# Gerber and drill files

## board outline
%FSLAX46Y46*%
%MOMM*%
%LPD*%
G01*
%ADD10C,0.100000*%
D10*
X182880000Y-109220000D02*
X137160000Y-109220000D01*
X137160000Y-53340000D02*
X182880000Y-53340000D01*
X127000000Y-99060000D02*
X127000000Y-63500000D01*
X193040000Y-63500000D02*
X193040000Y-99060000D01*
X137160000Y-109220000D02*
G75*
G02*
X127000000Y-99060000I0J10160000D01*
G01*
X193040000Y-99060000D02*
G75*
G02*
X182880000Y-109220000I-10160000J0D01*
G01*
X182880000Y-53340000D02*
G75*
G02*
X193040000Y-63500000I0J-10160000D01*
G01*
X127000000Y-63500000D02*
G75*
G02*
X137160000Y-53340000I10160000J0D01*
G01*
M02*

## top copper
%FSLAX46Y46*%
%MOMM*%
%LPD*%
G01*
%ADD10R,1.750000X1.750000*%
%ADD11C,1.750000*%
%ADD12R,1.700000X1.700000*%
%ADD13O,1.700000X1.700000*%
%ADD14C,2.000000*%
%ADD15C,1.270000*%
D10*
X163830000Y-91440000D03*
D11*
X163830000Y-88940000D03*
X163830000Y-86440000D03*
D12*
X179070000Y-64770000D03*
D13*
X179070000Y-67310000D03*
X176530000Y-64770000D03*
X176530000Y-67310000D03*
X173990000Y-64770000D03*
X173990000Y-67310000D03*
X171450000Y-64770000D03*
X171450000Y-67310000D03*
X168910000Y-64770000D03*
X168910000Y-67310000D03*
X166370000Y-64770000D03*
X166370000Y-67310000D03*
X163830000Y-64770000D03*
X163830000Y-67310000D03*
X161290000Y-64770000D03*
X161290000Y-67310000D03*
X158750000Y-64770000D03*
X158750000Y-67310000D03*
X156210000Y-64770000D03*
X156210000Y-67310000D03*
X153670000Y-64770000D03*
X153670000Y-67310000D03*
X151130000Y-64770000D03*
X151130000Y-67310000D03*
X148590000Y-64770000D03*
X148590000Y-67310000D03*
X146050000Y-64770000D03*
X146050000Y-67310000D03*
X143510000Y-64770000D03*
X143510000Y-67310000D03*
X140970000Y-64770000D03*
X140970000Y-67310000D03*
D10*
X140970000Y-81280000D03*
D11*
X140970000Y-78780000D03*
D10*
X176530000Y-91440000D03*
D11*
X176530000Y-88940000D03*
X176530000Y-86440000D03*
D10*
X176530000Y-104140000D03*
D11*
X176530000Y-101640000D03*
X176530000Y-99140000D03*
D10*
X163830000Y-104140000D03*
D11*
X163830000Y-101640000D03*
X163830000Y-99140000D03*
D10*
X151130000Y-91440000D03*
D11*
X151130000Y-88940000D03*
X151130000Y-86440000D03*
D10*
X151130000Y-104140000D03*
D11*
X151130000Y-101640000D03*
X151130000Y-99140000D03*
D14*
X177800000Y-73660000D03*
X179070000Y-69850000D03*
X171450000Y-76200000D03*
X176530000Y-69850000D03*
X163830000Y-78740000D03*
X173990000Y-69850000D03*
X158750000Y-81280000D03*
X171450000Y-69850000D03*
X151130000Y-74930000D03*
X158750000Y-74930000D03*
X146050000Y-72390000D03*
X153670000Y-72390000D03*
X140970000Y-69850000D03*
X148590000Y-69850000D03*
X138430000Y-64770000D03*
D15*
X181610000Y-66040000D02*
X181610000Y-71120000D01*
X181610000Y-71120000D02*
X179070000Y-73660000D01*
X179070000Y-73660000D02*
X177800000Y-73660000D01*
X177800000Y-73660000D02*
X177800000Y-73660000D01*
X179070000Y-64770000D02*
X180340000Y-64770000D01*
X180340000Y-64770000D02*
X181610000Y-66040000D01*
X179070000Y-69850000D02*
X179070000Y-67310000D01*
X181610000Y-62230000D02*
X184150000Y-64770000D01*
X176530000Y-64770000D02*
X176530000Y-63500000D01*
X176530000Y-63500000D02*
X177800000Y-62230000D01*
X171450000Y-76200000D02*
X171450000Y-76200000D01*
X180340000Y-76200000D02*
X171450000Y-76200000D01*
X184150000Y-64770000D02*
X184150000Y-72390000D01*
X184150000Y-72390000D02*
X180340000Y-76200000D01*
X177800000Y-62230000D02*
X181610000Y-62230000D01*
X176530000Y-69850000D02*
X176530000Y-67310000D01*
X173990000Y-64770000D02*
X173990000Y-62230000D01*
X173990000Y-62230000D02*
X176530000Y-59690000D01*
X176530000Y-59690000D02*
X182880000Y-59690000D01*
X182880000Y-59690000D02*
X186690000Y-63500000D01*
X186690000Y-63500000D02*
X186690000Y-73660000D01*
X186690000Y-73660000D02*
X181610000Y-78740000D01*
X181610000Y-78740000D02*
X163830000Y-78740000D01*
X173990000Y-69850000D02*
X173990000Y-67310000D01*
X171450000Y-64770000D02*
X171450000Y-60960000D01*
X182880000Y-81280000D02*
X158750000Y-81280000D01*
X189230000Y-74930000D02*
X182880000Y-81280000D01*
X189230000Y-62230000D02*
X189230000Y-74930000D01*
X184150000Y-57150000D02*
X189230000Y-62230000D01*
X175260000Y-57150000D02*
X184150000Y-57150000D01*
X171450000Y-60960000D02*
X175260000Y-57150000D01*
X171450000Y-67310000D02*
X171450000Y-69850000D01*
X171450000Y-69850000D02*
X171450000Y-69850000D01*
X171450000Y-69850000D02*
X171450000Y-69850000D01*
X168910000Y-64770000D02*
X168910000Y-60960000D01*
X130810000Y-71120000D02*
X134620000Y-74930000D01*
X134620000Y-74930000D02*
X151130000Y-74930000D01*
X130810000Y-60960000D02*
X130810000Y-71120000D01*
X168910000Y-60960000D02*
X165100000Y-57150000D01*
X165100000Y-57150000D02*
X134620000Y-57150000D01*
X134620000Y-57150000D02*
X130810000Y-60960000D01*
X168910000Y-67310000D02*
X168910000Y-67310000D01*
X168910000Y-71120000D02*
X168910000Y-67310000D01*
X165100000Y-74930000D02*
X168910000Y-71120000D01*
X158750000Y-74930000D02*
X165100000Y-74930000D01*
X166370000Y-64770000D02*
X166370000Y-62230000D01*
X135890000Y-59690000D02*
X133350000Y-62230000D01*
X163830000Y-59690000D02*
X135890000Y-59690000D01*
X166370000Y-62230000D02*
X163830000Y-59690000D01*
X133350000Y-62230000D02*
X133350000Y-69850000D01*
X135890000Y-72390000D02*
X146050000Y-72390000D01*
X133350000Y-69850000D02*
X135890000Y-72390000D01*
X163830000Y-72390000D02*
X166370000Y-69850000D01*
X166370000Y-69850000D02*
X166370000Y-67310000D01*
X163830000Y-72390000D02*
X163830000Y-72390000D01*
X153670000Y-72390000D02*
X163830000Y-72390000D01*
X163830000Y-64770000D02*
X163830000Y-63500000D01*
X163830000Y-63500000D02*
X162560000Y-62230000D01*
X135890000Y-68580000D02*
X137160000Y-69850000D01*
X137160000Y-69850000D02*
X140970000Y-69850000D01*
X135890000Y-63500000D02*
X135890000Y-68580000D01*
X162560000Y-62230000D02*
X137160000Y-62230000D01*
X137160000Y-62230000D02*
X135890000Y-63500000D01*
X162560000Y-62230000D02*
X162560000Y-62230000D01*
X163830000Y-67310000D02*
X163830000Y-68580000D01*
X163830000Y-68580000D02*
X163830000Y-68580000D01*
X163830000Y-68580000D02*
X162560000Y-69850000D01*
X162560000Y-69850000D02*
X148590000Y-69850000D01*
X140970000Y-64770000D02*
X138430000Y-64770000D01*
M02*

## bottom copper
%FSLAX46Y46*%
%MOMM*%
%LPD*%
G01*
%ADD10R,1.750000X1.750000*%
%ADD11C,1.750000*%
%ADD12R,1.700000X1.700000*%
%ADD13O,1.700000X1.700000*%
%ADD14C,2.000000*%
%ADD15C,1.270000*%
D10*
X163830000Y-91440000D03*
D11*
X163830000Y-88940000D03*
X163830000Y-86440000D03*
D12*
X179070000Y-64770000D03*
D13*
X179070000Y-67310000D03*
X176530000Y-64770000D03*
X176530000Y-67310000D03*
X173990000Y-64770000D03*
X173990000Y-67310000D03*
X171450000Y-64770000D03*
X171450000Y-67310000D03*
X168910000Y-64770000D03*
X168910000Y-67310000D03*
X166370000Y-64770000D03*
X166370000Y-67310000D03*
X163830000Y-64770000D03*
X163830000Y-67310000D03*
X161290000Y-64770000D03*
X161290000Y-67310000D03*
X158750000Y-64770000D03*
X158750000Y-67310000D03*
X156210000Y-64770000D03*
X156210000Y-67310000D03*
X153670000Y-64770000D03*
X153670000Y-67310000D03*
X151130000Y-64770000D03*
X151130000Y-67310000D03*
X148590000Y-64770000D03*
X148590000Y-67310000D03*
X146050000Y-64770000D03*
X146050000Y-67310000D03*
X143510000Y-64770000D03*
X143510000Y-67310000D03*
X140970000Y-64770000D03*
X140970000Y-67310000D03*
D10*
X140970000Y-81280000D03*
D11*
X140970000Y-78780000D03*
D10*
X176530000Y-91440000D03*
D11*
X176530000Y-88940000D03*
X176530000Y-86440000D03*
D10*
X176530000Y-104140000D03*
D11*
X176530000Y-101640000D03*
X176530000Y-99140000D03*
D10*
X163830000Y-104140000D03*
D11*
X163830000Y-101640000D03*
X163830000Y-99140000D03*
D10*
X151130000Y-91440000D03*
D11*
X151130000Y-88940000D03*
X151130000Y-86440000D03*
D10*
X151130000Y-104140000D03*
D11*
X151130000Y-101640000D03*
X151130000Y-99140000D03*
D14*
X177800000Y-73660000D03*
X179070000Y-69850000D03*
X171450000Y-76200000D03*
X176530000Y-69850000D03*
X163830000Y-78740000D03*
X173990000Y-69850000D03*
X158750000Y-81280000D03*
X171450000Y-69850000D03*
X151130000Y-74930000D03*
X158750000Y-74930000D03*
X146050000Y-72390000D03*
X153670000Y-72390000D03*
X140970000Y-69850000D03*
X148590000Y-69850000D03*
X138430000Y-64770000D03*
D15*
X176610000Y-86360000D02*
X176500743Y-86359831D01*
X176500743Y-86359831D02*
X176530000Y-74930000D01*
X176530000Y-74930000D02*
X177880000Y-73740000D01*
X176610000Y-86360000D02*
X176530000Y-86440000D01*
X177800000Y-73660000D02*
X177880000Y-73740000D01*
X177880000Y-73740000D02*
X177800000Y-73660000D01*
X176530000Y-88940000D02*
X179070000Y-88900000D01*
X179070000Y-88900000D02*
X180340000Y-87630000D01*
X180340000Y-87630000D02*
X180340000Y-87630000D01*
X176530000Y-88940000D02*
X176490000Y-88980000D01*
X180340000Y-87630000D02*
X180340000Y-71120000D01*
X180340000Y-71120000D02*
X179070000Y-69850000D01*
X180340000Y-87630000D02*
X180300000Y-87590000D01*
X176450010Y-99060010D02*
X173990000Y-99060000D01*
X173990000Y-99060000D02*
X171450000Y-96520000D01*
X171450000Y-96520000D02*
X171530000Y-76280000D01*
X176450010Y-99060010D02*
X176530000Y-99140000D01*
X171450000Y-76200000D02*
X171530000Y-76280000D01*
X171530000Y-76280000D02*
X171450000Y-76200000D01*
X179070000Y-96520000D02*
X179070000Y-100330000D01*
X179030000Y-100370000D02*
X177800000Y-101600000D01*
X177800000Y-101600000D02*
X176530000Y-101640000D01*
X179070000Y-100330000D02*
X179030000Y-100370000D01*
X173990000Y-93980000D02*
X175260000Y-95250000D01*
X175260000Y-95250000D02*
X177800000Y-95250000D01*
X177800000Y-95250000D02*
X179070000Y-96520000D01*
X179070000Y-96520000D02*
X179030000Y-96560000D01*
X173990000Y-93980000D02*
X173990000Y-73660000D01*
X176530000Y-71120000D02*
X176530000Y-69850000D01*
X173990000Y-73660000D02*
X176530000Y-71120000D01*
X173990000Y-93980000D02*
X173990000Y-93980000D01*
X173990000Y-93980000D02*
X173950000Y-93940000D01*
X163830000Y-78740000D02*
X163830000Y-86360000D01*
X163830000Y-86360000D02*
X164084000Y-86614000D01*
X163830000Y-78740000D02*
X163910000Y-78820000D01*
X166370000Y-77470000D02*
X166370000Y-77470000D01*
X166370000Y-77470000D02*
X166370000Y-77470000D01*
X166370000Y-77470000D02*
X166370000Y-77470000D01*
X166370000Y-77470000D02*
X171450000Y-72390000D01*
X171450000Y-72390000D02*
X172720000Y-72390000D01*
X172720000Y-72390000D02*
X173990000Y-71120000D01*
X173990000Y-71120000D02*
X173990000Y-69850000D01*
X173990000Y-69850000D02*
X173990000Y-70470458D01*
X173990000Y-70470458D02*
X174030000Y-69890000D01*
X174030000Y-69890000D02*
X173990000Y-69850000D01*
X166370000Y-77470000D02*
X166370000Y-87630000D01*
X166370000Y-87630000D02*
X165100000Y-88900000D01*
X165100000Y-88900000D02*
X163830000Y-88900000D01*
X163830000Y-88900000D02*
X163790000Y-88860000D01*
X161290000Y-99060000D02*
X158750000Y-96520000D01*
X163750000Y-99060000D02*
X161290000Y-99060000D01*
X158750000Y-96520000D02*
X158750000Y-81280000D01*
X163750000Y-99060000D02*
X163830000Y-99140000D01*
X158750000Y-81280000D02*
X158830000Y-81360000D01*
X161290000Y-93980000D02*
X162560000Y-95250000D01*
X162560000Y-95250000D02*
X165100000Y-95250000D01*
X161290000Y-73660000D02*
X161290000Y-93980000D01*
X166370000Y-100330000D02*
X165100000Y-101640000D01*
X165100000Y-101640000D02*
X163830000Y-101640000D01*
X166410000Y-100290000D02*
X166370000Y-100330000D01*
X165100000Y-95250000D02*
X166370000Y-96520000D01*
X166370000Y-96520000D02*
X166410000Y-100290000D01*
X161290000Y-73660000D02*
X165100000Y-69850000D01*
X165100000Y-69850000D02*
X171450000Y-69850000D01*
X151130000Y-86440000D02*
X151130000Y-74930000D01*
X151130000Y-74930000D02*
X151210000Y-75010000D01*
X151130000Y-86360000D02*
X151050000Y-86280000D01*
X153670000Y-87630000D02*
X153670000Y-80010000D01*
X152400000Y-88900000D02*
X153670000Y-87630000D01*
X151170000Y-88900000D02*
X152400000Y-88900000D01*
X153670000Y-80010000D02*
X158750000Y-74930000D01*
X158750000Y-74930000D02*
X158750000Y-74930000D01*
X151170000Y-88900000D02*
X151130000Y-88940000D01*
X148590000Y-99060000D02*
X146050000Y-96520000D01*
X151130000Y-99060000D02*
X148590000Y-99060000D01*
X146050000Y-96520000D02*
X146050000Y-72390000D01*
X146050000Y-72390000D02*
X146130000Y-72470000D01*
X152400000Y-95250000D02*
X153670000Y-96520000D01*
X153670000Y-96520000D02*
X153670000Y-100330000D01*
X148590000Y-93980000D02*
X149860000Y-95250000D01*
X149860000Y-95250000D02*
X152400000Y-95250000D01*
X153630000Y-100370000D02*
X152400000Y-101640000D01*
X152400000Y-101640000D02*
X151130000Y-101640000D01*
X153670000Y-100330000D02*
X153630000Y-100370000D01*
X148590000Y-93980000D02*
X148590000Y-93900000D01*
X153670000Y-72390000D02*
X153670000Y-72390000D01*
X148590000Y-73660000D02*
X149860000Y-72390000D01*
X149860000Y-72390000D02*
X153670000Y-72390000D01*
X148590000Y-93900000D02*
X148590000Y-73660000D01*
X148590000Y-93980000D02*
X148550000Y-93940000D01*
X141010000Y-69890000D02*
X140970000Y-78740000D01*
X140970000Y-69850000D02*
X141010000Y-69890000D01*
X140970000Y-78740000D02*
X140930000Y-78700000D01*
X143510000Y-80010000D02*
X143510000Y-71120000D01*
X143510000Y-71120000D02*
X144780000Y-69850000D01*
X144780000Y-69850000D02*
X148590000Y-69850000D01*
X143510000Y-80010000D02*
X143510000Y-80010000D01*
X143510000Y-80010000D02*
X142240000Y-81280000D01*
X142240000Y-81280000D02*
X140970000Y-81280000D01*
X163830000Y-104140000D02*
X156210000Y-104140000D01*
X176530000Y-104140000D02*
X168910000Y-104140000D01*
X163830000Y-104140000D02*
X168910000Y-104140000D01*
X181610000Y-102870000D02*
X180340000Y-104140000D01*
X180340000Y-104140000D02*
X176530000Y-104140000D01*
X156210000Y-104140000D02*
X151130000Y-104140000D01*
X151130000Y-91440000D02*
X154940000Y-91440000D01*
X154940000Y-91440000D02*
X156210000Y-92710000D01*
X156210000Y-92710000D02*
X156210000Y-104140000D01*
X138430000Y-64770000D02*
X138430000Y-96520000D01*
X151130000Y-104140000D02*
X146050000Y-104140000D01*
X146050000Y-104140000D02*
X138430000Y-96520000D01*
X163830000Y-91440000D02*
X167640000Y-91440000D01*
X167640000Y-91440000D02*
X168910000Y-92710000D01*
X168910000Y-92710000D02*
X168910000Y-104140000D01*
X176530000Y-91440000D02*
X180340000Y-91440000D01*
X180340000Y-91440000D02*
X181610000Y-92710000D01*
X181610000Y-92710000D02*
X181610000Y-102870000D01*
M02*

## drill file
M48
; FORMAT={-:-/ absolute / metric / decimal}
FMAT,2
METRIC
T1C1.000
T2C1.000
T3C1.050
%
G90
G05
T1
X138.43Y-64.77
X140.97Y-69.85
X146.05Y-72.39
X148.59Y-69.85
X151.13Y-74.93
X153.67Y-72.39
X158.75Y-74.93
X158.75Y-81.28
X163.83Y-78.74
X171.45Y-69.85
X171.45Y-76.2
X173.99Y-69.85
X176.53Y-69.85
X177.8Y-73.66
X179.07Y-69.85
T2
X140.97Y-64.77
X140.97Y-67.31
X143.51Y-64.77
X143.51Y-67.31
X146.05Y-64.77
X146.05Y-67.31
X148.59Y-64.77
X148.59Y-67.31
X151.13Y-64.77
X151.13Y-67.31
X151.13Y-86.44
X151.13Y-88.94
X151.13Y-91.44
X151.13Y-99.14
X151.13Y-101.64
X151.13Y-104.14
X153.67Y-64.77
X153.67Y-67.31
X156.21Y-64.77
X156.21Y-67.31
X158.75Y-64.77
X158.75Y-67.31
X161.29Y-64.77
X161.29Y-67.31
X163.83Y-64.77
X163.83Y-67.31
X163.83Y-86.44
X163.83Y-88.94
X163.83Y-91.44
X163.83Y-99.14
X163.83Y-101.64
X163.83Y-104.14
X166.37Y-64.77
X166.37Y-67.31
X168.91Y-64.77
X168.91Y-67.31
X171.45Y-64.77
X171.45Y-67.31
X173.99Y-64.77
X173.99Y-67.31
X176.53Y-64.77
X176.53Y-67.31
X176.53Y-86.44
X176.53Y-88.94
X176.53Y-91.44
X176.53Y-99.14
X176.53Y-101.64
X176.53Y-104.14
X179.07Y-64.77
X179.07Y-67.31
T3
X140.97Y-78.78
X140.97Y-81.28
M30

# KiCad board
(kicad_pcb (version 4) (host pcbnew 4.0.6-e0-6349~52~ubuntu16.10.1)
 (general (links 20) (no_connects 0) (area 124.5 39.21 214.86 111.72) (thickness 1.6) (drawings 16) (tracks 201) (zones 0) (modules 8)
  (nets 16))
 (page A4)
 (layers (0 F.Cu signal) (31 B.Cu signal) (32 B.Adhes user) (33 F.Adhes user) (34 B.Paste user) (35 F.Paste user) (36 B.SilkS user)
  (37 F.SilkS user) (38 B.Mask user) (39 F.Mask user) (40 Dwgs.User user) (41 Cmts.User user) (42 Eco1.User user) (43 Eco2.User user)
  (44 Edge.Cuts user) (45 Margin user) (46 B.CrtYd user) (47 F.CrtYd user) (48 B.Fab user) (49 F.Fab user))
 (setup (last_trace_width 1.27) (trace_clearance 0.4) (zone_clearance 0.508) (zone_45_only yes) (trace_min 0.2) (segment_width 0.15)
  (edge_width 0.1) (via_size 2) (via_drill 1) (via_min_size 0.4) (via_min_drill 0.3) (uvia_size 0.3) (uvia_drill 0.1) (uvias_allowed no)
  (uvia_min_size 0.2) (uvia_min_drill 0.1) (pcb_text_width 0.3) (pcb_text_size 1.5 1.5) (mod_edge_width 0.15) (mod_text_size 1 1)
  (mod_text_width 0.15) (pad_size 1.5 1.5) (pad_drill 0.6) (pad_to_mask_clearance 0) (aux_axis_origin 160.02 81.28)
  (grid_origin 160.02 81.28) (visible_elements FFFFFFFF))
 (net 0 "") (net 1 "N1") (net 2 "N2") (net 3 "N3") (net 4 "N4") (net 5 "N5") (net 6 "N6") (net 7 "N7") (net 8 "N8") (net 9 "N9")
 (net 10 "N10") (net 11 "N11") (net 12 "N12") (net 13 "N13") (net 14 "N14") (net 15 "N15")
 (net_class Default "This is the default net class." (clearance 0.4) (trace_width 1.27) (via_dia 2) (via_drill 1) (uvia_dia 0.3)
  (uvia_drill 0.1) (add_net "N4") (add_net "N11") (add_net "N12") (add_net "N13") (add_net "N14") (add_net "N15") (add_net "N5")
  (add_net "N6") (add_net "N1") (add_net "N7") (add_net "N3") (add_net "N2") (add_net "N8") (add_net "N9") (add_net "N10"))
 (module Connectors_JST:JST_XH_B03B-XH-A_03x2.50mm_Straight (layer F.Cu) (at 163.83 91.44 90)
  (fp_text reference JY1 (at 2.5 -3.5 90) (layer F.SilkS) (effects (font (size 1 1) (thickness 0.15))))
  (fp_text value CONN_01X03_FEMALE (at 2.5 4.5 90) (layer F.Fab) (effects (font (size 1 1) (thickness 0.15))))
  (pad 1 thru_hole rect (at 0 0 90) (size 1.75 1.75) (drill 1) (layers *.Cu *.Mask) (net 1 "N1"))
  (pad 2 thru_hole circle (at 2.5 0 90) (size 1.75 1.75) (drill 1) (layers *.Cu *.Mask) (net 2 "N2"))
  (pad 3 thru_hole circle (at 5 0 90) (size 1.75 1.75) (drill 1) (layers *.Cu *.Mask) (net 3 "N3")))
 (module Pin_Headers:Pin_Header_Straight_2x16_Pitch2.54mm (layer F.Cu) (at 179.07 64.77 270)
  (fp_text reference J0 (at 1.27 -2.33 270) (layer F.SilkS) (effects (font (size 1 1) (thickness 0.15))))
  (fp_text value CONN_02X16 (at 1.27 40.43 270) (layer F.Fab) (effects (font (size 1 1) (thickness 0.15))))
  (pad 1 thru_hole rect (at 0 0 270) (size 1.7 1.7) (drill 1) (layers *.Cu *.Mask) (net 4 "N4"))
  (pad 2 thru_hole oval (at 2.54 0 270) (size 1.7 1.7) (drill 1) (layers *.Cu *.Mask) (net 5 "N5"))
  (pad 3 thru_hole oval (at 0 2.54 270) (size 1.7 1.7) (drill 1) (layers *.Cu *.Mask) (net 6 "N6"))
  (pad 4 thru_hole oval (at 2.54 2.54 270) (size 1.7 1.7) (drill 1) (layers *.Cu *.Mask) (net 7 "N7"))
  (pad 5 thru_hole oval (at 0 5.08 270) (size 1.7 1.7) (drill 1) (layers *.Cu *.Mask) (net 3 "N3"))
  (pad 6 thru_hole oval (at 2.54 5.08 270) (size 1.7 1.7) (drill 1) (layers *.Cu *.Mask) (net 2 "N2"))
  (pad 7 thru_hole oval (at 0 7.62 270) (size 1.7 1.7) (drill 1) (layers *.Cu *.Mask) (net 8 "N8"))
  (pad 8 thru_hole oval (at 2.54 7.62 270) (size 1.7 1.7) (drill 1) (layers *.Cu *.Mask) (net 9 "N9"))
  (pad 9 thru_hole oval (at 0 10.16 270) (size 1.7 1.7) (drill 1) (layers *.Cu *.Mask) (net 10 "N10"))
  (pad 10 thru_hole oval (at 2.54 10.16 270) (size 1.7 1.7) (drill 1) (layers *.Cu *.Mask) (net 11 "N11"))
  (pad 11 thru_hole oval (at 0 12.7 270) (size 1.7 1.7) (drill 1) (layers *.Cu *.Mask) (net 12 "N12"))
  (pad 12 thru_hole oval (at 2.54 12.7 270) (size 1.7 1.7) (drill 1) (layers *.Cu *.Mask) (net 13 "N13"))
  (pad 13 thru_hole oval (at 0 15.24 270) (size 1.7 1.7) (drill 1) (layers *.Cu *.Mask) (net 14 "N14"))
  (pad 14 thru_hole oval (at 2.54 15.24 270) (size 1.7 1.7) (drill 1) (layers *.Cu *.Mask) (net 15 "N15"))
  (pad 15 thru_hole oval (at 0 17.78 270) (size 1.7 1.7) (drill 1) (layers *.Cu *.Mask))
  (pad 16 thru_hole oval (at 2.54 17.78 270) (size 1.7 1.7) (drill 1) (layers *.Cu *.Mask))
  (pad 17 thru_hole oval (at 0 20.32 270) (size 1.7 1.7) (drill 1) (layers *.Cu *.Mask))
  (pad 18 thru_hole oval (at 2.54 20.32 270) (size 1.7 1.7) (drill 1) (layers *.Cu *.Mask))
  (pad 19 thru_hole oval (at 0 22.86 270) (size 1.7 1.7) (drill 1) (layers *.Cu *.Mask))
  (pad 20 thru_hole oval (at 2.54 22.86 270) (size 1.7 1.7) (drill 1) (layers *.Cu *.Mask))
  (pad 21 thru_hole oval (at 0 25.4 270) (size 1.7 1.7) (drill 1) (layers *.Cu *.Mask))
  (pad 22 thru_hole oval (at 2.54 25.4 270) (size 1.7 1.7) (drill 1) (layers *.Cu *.Mask))
  (pad 23 thru_hole oval (at 0 27.94 270) (size 1.7 1.7) (drill 1) (layers *.Cu *.Mask))
  (pad 24 thru_hole oval (at 2.54 27.94 270) (size 1.7 1.7) (drill 1) (layers *.Cu *.Mask))
  (pad 25 thru_hole oval (at 0 30.48 270) (size 1.7 1.7) (drill 1) (layers *.Cu *.Mask))
  (pad 26 thru_hole oval (at 2.54 30.48 270) (size 1.7 1.7) (drill 1) (layers *.Cu *.Mask))
  (pad 27 thru_hole oval (at 0 33.02 270) (size 1.7 1.7) (drill 1) (layers *.Cu *.Mask))
  (pad 28 thru_hole oval (at 2.54 33.02 270) (size 1.7 1.7) (drill 1) (layers *.Cu *.Mask))
  (pad 29 thru_hole oval (at 0 35.56 270) (size 1.7 1.7) (drill 1) (layers *.Cu *.Mask))
  (pad 30 thru_hole oval (at 2.54 35.56 270) (size 1.7 1.7) (drill 1) (layers *.Cu *.Mask))
  (pad 31 thru_hole oval (at 0 38.1 270) (size 1.7 1.7) (drill 1) (layers *.Cu *.Mask) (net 1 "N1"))
  (pad 32 thru_hole oval (at 2.54 38.1 270) (size 1.7 1.7) (drill 1) (layers *.Cu *.Mask)))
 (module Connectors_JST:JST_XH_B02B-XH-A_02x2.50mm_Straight (layer F.Cu) (at 140.97 81.28 90)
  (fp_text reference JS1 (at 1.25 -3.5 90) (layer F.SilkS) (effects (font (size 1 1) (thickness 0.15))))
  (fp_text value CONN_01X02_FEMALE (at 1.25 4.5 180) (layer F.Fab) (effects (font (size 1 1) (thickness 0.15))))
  (pad 1 thru_hole rect (at 0 0 90) (size 1.75 1.75) (drill 1.05) (layers *.Cu *.Mask) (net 15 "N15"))
  (pad 2 thru_hole circle (at 2.5 0 90) (size 1.75 1.75) (drill 1.05) (layers *.Cu *.Mask) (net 14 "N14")))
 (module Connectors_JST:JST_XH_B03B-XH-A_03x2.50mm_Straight (layer F.Cu) (at 176.53 91.44 90)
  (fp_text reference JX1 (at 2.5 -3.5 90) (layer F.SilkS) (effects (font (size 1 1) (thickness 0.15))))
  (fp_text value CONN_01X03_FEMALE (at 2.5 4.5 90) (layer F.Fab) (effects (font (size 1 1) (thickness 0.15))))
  (pad 1 thru_hole rect (at 0 0 90) (size 1.75 1.75) (drill 1) (layers *.Cu *.Mask) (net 1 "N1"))
  (pad 2 thru_hole circle (at 2.5 0 90) (size 1.75 1.75) (drill 1) (layers *.Cu *.Mask) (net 5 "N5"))
  (pad 3 thru_hole circle (at 5 0 90) (size 1.75 1.75) (drill 1) (layers *.Cu *.Mask) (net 4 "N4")))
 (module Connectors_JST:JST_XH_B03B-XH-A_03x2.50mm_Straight (layer F.Cu) (at 176.53 104.14 90)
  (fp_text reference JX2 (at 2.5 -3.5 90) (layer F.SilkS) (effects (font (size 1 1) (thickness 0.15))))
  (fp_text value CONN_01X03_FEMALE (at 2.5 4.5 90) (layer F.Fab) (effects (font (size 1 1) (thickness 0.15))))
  (pad 1 thru_hole rect (at 0 0 90) (size 1.75 1.75) (drill 1) (layers *.Cu *.Mask) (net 1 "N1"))
  (pad 2 thru_hole circle (at 2.5 0 90) (size 1.75 1.75) (drill 1) (layers *.Cu *.Mask) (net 7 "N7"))
  (pad 3 thru_hole circle (at 5 0 90) (size 1.75 1.75) (drill 1) (layers *.Cu *.Mask) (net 6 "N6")))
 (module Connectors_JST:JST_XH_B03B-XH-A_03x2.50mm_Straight (layer F.Cu) (at 163.83 104.14 90)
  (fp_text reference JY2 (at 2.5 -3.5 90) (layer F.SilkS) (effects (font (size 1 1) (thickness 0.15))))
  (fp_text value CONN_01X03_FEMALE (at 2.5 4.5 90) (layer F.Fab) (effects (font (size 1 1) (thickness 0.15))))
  (pad 1 thru_hole rect (at 0 0 90) (size 1.75 1.75) (drill 1) (layers *.Cu *.Mask) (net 1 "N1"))
  (pad 2 thru_hole circle (at 2.5 0 90) (size 1.75 1.75) (drill 1) (layers *.Cu *.Mask) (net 9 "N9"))
  (pad 3 thru_hole circle (at 5 0 90) (size 1.75 1.75) (drill 1) (layers *.Cu *.Mask) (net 8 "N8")))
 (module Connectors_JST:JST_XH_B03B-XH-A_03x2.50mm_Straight (layer F.Cu) (at 151.13 91.44 90)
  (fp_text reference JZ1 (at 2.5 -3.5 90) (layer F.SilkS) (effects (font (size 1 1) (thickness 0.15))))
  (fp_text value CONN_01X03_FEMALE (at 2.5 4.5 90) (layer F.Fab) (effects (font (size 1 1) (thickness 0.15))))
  (pad 1 thru_hole rect (at 0 0 90) (size 1.75 1.75) (drill 1) (layers *.Cu *.Mask) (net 1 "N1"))
  (pad 2 thru_hole circle (at 2.5 0 90) (size 1.75 1.75) (drill 1) (layers *.Cu *.Mask) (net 11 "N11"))
  (pad 3 thru_hole circle (at 5 0 90) (size 1.75 1.75) (drill 1) (layers *.Cu *.Mask) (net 10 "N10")))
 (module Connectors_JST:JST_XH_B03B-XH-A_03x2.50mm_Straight (layer F.Cu) (at 151.13 104.14 90)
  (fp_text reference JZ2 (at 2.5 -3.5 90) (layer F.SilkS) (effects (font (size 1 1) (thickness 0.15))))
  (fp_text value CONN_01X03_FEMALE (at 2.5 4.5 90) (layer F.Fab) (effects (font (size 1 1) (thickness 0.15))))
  (pad 1 thru_hole rect (at 0 0 90) (size 1.75 1.75) (drill 1) (layers *.Cu *.Mask) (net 1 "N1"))
  (pad 2 thru_hole circle (at 2.5 0 90) (size 1.75 1.75) (drill 1) (layers *.Cu *.Mask) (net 13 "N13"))
  (pad 3 thru_hole circle (at 5 0 90) (size 1.75 1.75) (drill 1) (layers *.Cu *.Mask) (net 12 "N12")))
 (gr_line (start 182.88 109.22) (end 137.16 109.22) (angle 90) (layer Edge.Cuts) (width 0.1))
 (gr_line (start 137.16 53.34) (end 182.88 53.34) (angle 90) (layer Edge.Cuts) (width 0.1))
 (gr_line (start 127 99.06) (end 127 63.5) (angle 90) (layer Edge.Cuts) (width 0.1))
 (gr_line (start 193.04 63.5) (end 193.04 99.06) (angle 90) (layer Edge.Cuts) (width 0.1))
 (gr_arc (start 137.16 99.06) (end 137.16 109.22) (angle 90) (layer Edge.Cuts) (width 0.1))
 (gr_arc (start 182.88 99.06) (end 193.04 99.06) (angle 90) (layer Edge.Cuts) (width 0.1))
 (gr_arc (start 182.88 63.5) (end 182.88 53.34) (angle 90) (layer Edge.Cuts) (width 0.1))
 (gr_arc (start 137.16 63.5) (end 127 63.5) (angle 90) (layer Edge.Cuts) (width 0.1))
 (segment (start 176.61 86.36) (end 176.500743 86.359831) (width 1.27) (layer B.Cu) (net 4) (status 30))
 (segment (start 176.500743 86.359831) (end 176.53 74.93) (width 1.27) (layer B.Cu) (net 4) (status 10))
 (segment (start 176.53 74.93) (end 177.88 73.74) (width 1.27) (layer B.Cu) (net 4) (status 10))
 (segment (start 176.61 86.36) (end 176.53 86.44) (width 1.27) (layer B.Cu) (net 4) (status 30))
 (via (at 177.8 73.66) (size 2) (drill 1) (layers F.Cu B.Cu) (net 4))
 (segment (start 181.61 66.04) (end 181.61 71.12) (width 1.27) (layer F.Cu) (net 4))
 (segment (start 181.61 71.12) (end 179.07 73.66) (width 1.27) (layer F.Cu) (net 4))
 (segment (start 179.07 73.66) (end 177.8 73.66) (width 1.27) (layer F.Cu) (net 4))
 (segment (start 177.8 73.66) (end 177.8 73.66) (width 1.27) (layer F.Cu) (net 4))
 (segment (start 179.07 64.77) (end 180.34 64.77) (width 1.27) (layer F.Cu) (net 4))
 (segment (start 180.34 64.77) (end 181.61 66.04) (width 1.27) (layer F.Cu) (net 4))
 (segment (start 177.8 73.66) (end 177.88 73.74) (width 1.27) (layer B.Cu) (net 4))
 (segment (start 177.88 73.74) (end 177.8 73.66) (width 1.27) (layer B.Cu) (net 4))
 (segment (start 176.53 88.94) (end 179.07 88.9) (width 1.27) (layer B.Cu) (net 5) (status 10))
 (segment (start 179.07 88.9) (end 180.34 87.63) (width 1.27) (layer B.Cu) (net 5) (status 10))
 (segment (start 180.34 87.63) (end 180.34 87.63) (width 1.27) (layer B.Cu) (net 5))
 (segment (start 176.53 88.94) (end 176.49 88.98) (width 1.27) (layer B.Cu) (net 5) (status 30))
 (segment (start 180.34 87.63) (end 180.34 71.12) (width 1.27) (layer B.Cu) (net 5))
 (segment (start 180.34 71.12) (end 179.07 69.85) (width 1.27) (layer B.Cu) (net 5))
 (via (at 179.07 69.85) (size 2) (drill 1) (layers F.Cu B.Cu) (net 5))
 (segment (start 179.07 69.85) (end 179.07 67.31) (width 1.27) (layer F.Cu) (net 5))
 (segment (start 180.34 87.63) (end 180.3 87.59) (width 1.27) (layer B.Cu) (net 5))
 (segment (start 181.61 62.23) (end 184.15 64.77) (width 1.27) (layer F.Cu) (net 6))
 (segment (start 176.45001 99.06001) (end 173.99 99.06) (width 1.27) (layer B.Cu) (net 6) (status 10))
 (segment (start 173.99 99.06) (end 171.45 96.52) (width 1.27) (layer B.Cu) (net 6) (status 10))
 (segment (start 171.45 96.52) (end 171.53 76.28) (width 1.27) (layer B.Cu) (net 6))
 (segment (start 176.45001 99.06001) (end 176.53 99.14) (width 1.27) (layer B.Cu) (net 6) (status 30))
 (segment (start 176.53 64.77) (end 176.53 63.5) (width 1.27) (layer F.Cu) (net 6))
 (segment (start 176.53 63.5) (end 177.8 62.23) (width 1.27) (layer F.Cu) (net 6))
 (via (at 171.45 76.2) (size 2) (drill 1) (layers F.Cu B.Cu) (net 6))
 (segment (start 171.45 76.2) (end 171.45 76.2) (width 1.27) (layer F.Cu) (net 6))
 (segment (start 180.34 76.2) (end 171.45 76.2) (width 1.27) (layer F.Cu) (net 6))
 (segment (start 184.15 64.77) (end 184.15 72.39) (width 1.27) (layer F.Cu) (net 6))
 (segment (start 184.15 72.39) (end 180.34 76.2) (width 1.27) (layer F.Cu) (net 6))
 (segment (start 177.8 62.23) (end 181.61 62.23) (width 1.27) (layer F.Cu) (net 6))
 (segment (start 171.45 76.2) (end 171.53 76.28) (width 1.27) (layer B.Cu) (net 6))
 (segment (start 171.53 76.28) (end 171.45 76.2) (width 1.27) (layer B.Cu) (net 6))
 (segment (start 179.07 96.52) (end 179.07 100.33) (width 1.27) (layer B.Cu) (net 7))
 (segment (start 179.03 100.37) (end 177.8 101.6) (width 1.27) (layer B.Cu) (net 7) (status 20))
 (segment (start 177.8 101.6) (end 176.53 101.64) (width 1.27) (layer B.Cu) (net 7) (status 20))
 (segment (start 179.07 100.33) (end 179.03 100.37) (width 1.27) (layer B.Cu) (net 7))
 (segment (start 173.99 93.98) (end 175.26 95.25) (width 1.27) (layer B.Cu) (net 7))
 (segment (start 175.26 95.25) (end 177.8 95.25) (width 1.27) (layer B.Cu) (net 7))
 (segment (start 177.8 95.25) (end 179.07 96.52) (width 1.27) (layer B.Cu) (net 7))
 (segment (start 179.07 96.52) (end 179.03 96.56) (width 1.27) (layer B.Cu) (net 7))
 (segment (start 173.99 93.98) (end 173.99 73.66) (width 1.27) (layer B.Cu) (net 7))
 (segment (start 176.53 69.85) (end 176.53 67.31) (width 1.27) (layer F.Cu) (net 7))
 (via (at 176.53 69.85) (size 2) (drill 1) (layers F.Cu B.Cu) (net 7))
 (segment (start 176.53 71.12) (end 176.53 69.85) (width 1.27) (layer B.Cu) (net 7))
 (segment (start 173.99 73.66) (end 176.53 71.12) (width 1.27) (layer B.Cu) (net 7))
 (segment (start 173.99 93.98) (end 173.99 93.98) (width 1.27) (layer B.Cu) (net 7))
 (segment (start 173.99 93.98) (end 173.95 93.94) (width 1.27) (layer B.Cu) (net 7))
 (segment (start 163.83 78.74) (end 163.83 86.36) (width 1.27) (layer B.Cu) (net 3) (status 20))
 (segment (start 163.83 86.36) (end 164.084 86.614) (width 1.27) (layer B.Cu) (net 3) (status 30))
 (segment (start 173.99 64.77) (end 173.99 62.23) (width 1.27) (layer F.Cu) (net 3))
 (segment (start 173.99 62.23) (end 176.53 59.69) (width 1.27) (layer F.Cu) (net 3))
 (segment (start 176.53 59.69) (end 182.88 59.69) (width 1.27) (layer F.Cu) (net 3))
 (segment (start 182.88 59.69) (end 186.69 63.5) (width 1.27) (layer F.Cu) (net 3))
 (segment (start 186.69 63.5) (end 186.69 73.66) (width 1.27) (layer F.Cu) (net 3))
 (segment (start 186.69 73.66) (end 181.61 78.74) (width 1.27) (layer F.Cu) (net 3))
 (segment (start 181.61 78.74) (end 163.83 78.74) (width 1.27) (layer F.Cu) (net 3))
 (via (at 163.83 78.74) (size 2) (drill 1) (layers F.Cu B.Cu) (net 3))
 (segment (start 163.83 78.74) (end 163.91 78.82) (width 1.27) (layer B.Cu) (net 3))
 (segment (start 166.37 77.47) (end 166.37 77.47) (width 1.27) (layer B.Cu) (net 2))
 (segment (start 166.37 77.47) (end 166.37 77.47) (width 1.27) (layer B.Cu) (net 2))
 (segment (start 166.37 77.47) (end 166.37 77.47) (width 1.27) (layer B.Cu) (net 2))
 (segment (start 166.37 77.47) (end 171.45 72.39) (width 1.27) (layer B.Cu) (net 2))
 (segment (start 171.45 72.39) (end 172.72 72.39) (width 1.27) (layer B.Cu) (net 2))
 (segment (start 172.72 72.39) (end 173.99 71.12) (width 1.27) (layer B.Cu) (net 2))
 (segment (start 173.99 71.12) (end 173.99 69.85) (width 1.27) (layer B.Cu) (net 2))
 (segment (start 173.99 69.85) (end 173.99 70.470458) (width 1.27) (layer B.Cu) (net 2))
 (segment (start 173.99 70.470458) (end 174.03 69.89) (width 1.27) (layer B.Cu) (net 2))
 (segment (start 173.99 69.85) (end 173.99 67.31) (width 1.27) (layer F.Cu) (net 2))
 (via (at 173.99 69.85) (size 2) (drill 1) (layers F.Cu B.Cu) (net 2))
 (segment (start 174.03 69.89) (end 173.99 69.85) (width 1.27) (layer B.Cu) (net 2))
 (segment (start 166.37 77.47) (end 166.37 87.63) (width 1.27) (layer B.Cu) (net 2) (status 20))
 (segment (start 166.37 87.63) (end 165.1 88.9) (width 1.27) (layer B.Cu) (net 2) (status 20))
 (segment (start 165.1 88.9) (end 163.83 88.9) (width 1.27) (layer B.Cu) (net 2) (status 20))
 (segment (start 163.83 88.9) (end 163.79 88.86) (width 1.27) (layer B.Cu) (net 2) (status 30))
 (segment (start 161.29 99.06) (end 158.75 96.52) (width 1.27) (layer B.Cu) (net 8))
 (segment (start 163.75 99.06) (end 161.29 99.06) (width 1.27) (layer B.Cu) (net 8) (status 10))
 (segment (start 158.75 96.52) (end 158.75 81.28) (width 1.27) (layer B.Cu) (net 8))
 (segment (start 163.75 99.06) (end 163.83 99.14) (width 1.27) (layer B.Cu) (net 8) (status 30))
 (segment (start 171.45 64.77) (end 171.45 60.96) (width 1.27) (layer F.Cu) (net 8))
 (via (at 158.75 81.28) (size 2) (drill 1) (layers F.Cu B.Cu) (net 8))
 (segment (start 182.88 81.28) (end 158.75 81.28) (width 1.27) (layer F.Cu) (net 8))
 (segment (start 189.23 74.93) (end 182.88 81.28) (width 1.27) (layer F.Cu) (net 8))
 (segment (start 189.23 62.23) (end 189.23 74.93) (width 1.27) (layer F.Cu) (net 8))
 (segment (start 184.15 57.15) (end 189.23 62.23) (width 1.27) (layer F.Cu) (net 8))
 (segment (start 175.26 57.15) (end 184.15 57.15) (width 1.27) (layer F.Cu) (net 8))
 (segment (start 171.45 60.96) (end 175.26 57.15) (width 1.27) (layer F.Cu) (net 8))
 (segment (start 158.75 81.28) (end 158.83 81.36) (width 1.27) (layer B.Cu) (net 8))
 (segment (start 171.45 67.31) (end 171.45 69.85) (width 1.27) (layer F.Cu) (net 9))
 (segment (start 161.29 93.98) (end 162.56 95.25) (width 1.27) (layer B.Cu) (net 9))
 (segment (start 162.56 95.25) (end 165.1 95.25) (width 1.27) (layer B.Cu) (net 9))
 (segment (start 161.29 73.66) (end 161.29 93.98) (width 1.27) (layer B.Cu) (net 9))
 (segment (start 166.37 100.33) (end 165.1 101.64) (width 1.27) (layer B.Cu) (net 9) (status 20))
 (segment (start 165.1 101.64) (end 163.83 101.64) (width 1.27) (layer B.Cu) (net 9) (status 20))
 (segment (start 166.41 100.29) (end 166.37 100.33) (width 1.27) (layer B.Cu) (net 9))
 (segment (start 165.1 95.25) (end 166.37 96.52) (width 1.27) (layer B.Cu) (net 9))
 (segment (start 166.37 96.52) (end 166.41 100.29) (width 1.27) (layer B.Cu) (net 9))
 (segment (start 171.45 69.85) (end 171.45 69.85) (width 1.27) (layer F.Cu) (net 9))
 (segment (start 171.45 69.85) (end 171.45 69.85) (width 1.27) (layer F.Cu) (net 9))
 (via (at 171.45 69.85) (size 2) (drill 1) (layers F.Cu B.Cu) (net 9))
 (segment (start 161.29 73.66) (end 165.1 69.85) (width 1.27) (layer B.Cu) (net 9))
 (segment (start 165.1 69.85) (end 171.45 69.85) (width 1.27) (layer B.Cu) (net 9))
 (segment (start 151.13 86.44) (end 151.13 74.93) (width 1.27) (layer B.Cu) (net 10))
 (segment (start 168.91 64.77) (end 168.91 60.96) (width 1.27) (layer F.Cu) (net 10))
 (segment (start 151.13 74.93) (end 151.21 75.01) (width 1.27) (layer B.Cu) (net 10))
 (via (at 151.13 74.93) (size 2) (drill 1) (layers F.Cu B.Cu) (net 10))
 (segment (start 130.81 71.12) (end 134.62 74.93) (width 1.27) (layer F.Cu) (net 10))
 (segment (start 134.62 74.93) (end 151.13 74.93) (width 1.27) (layer F.Cu) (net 10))
 (segment (start 130.81 60.96) (end 130.81 71.12) (width 1.27) (layer F.Cu) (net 10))
 (segment (start 168.91 60.96) (end 165.1 57.15) (width 1.27) (layer F.Cu) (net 10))
 (segment (start 165.1 57.15) (end 134.62 57.15) (width 1.27) (layer F.Cu) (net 10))
 (segment (start 134.62 57.15) (end 130.81 60.96) (width 1.27) (layer F.Cu) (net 10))
 (segment (start 151.13 86.36) (end 151.05 86.28) (width 1.27) (layer B.Cu) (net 10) (status 30))
 (segment (start 153.67 87.63) (end 153.67 80.01) (width 1.27) (layer B.Cu) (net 11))
 (segment (start 152.4 88.9) (end 153.67 87.63) (width 1.27) (layer B.Cu) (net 11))
 (segment (start 151.17 88.9) (end 152.4 88.9) (width 1.27) (layer B.Cu) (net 11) (status 10))
 (segment (start 153.67 80.01) (end 158.75 74.93) (width 1.27) (layer B.Cu) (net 11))
 (segment (start 168.91 67.31) (end 168.91 67.31) (width 1.27) (layer F.Cu) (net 11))
 (segment (start 168.91 71.12) (end 168.91 67.31) (width 1.27) (layer F.Cu) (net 11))
 (via (at 158.75 74.93) (size 2) (drill 1) (layers F.Cu B.Cu) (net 11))
 (segment (start 165.1 74.93) (end 168.91 71.12) (width 1.27) (layer F.Cu) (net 11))
 (segment (start 158.75 74.93) (end 165.1 74.93) (width 1.27) (layer F.Cu) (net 11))
 (segment (start 158.75 74.93) (end 158.75 74.93) (width 1.27) (layer B.Cu) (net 11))
 (segment (start 151.17 88.9) (end 151.13 88.94) (width 1.27) (layer B.Cu) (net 11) (status 30))
 (segment (start 148.59 99.06) (end 146.05 96.52) (width 1.27) (layer B.Cu) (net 12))
 (segment (start 151.13 99.06) (end 148.59 99.06) (width 1.27) (layer B.Cu) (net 12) (status 10))
 (segment (start 146.05 96.52) (end 146.05 72.39) (width 1.27) (layer B.Cu) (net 12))
 (segment (start 166.37 64.77) (end 166.37 62.23) (width 1.27) (layer F.Cu) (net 12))
 (segment (start 135.89 59.69) (end 133.35 62.23) (width 1.27) (layer F.Cu) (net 12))
 (segment (start 163.83 59.69) (end 135.89 59.69) (width 1.27) (layer F.Cu) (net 12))
 (segment (start 166.37 62.23) (end 163.83 59.69) (width 1.27) (layer F.Cu) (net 12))
 (segment (start 133.35 62.23) (end 133.35 69.85) (width 1.27) (layer F.Cu) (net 12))
 (segment (start 135.89 72.39) (end 146.05 72.39) (width 1.27) (layer F.Cu) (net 12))
 (segment (start 133.35 69.85) (end 135.89 72.39) (width 1.27) (layer F.Cu) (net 12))
 (via (at 146.05 72.39) (size 2) (drill 1) (layers F.Cu B.Cu) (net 12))
 (segment (start 146.05 72.39) (end 146.13 72.47) (width 1.27) (layer B.Cu) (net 12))
 (segment (start 163.83 72.39) (end 166.37 69.85) (width 1.27) (layer F.Cu) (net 13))
 (segment (start 166.37 69.85) (end 166.37 67.31) (width 1.27) (layer F.Cu) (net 13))
 (segment (start 163.83 72.39) (end 163.83 72.39) (width 1.27) (layer F.Cu) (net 13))
 (via (at 153.67 72.39) (size 2) (drill 1) (layers F.Cu B.Cu) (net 13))
 (segment (start 153.67 72.39) (end 163.83 72.39) (width 1.27) (layer F.Cu) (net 13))
 (segment (start 152.4 95.25) (end 153.67 96.52) (width 1.27) (layer B.Cu) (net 13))
 (segment (start 153.67 96.52) (end 153.67 100.33) (width 1.27) (layer B.Cu) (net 13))
 (segment (start 148.59 93.98) (end 149.86 95.25) (width 1.27) (layer B.Cu) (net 13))
 (segment (start 149.86 95.25) (end 152.4 95.25) (width 1.27) (layer B.Cu) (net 13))
 (segment (start 153.63 100.37) (end 152.4 101.64) (width 1.27) (layer B.Cu) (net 13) (status 20))
 (segment (start 152.4 101.64) (end 151.13 101.64) (width 1.27) (layer B.Cu) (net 13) (status 20))
 (segment (start 153.67 100.33) (end 153.63 100.37) (width 1.27) (layer B.Cu) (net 13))
 (segment (start 148.59 93.98) (end 148.59 93.9) (width 1.27) (layer B.Cu) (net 13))
 (segment (start 153.67 72.39) (end 153.67 72.39) (width 1.27) (layer B.Cu) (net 13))
 (segment (start 148.59 73.66) (end 149.86 72.39) (width 1.27) (layer B.Cu) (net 13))
 (segment (start 149.86 72.39) (end 153.67 72.39) (width 1.27) (layer B.Cu) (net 13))
 (segment (start 148.59 93.9) (end 148.59 73.66) (width 1.27) (layer B.Cu) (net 13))
 (segment (start 148.59 93.98) (end 148.55 93.94) (width 1.27) (layer B.Cu) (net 13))
 (segment (start 163.83 64.77) (end 163.83 63.5) (width 1.27) (layer F.Cu) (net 14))
 (segment (start 163.83 63.5) (end 162.56 62.23) (width 1.27) (layer F.Cu) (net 14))
 (segment (start 141.01 69.89) (end 140.97 78.74) (width 1.27) (layer B.Cu) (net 14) (status 20))
 (segment (start 140.97 69.85) (end 141.01 69.89) (width 1.27) (layer B.Cu) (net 14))
 (via (at 140.97 69.85) (size 2) (drill 1) (layers F.Cu B.Cu) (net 14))
 (segment (start 135.89 68.58) (end 137.16 69.85) (width 1.27) (layer F.Cu) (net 14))
 (segment (start 137.16 69.85) (end 140.97 69.85) (width 1.27) (layer F.Cu) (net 14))
 (segment (start 135.89 63.5) (end 135.89 68.58) (width 1.27) (layer F.Cu) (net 14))
 (segment (start 162.56 62.23) (end 137.16 62.23) (width 1.27) (layer F.Cu) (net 14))
 (segment (start 137.16 62.23) (end 135.89 63.5) (width 1.27) (layer F.Cu) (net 14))
 (segment (start 162.56 62.23) (end 162.56 62.23) (width 1.27) (layer F.Cu) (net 14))
 (segment (start 140.97 78.74) (end 140.93 78.7) (width 1.27) (layer B.Cu) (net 14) (status 30))
 (segment (start 163.83 67.31) (end 163.83 68.58) (width 1.27) (layer F.Cu) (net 15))
 (segment (start 163.83 68.58) (end 163.83 68.58) (width 1.27) (layer F.Cu) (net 15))
 (segment (start 163.83 68.58) (end 162.56 69.85) (width 1.27) (layer F.Cu) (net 15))
 (segment (start 162.56 69.85) (end 148.59 69.85) (width 1.27) (layer F.Cu) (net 15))
 (segment (start 143.51 80.01) (end 143.51 71.12) (width 1.27) (layer B.Cu) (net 15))
 (segment (start 143.51 71.12) (end 144.78 69.85) (width 1.27) (layer B.Cu) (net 15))
 (segment (start 144.78 69.85) (end 148.59 69.85) (width 1.27) (layer B.Cu) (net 15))
 (via (at 148.59 69.85) (size 2) (drill 1) (layers F.Cu B.Cu) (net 15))
 (segment (start 143.51 80.01) (end 143.51 80.01) (width 1.27) (layer B.Cu) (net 15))
 (segment (start 143.51 80.01) (end 142.24 81.28) (width 1.27) (layer B.Cu) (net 15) (status 20))
 (segment (start 142.24 81.28) (end 140.97 81.28) (width 1.27) (layer B.Cu) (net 15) (status 20))
 (segment (start 163.83 104.14) (end 156.21 104.14) (width 1.27) (layer B.Cu) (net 1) (status 10))
 (segment (start 176.53 104.14) (end 168.91 104.14) (width 1.27) (layer B.Cu) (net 1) (status 10))
 (segment (start 163.83 104.14) (end 168.91 104.14) (width 1.27) (layer B.Cu) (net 1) (status 10))
 (segment (start 181.61 102.87) (end 180.34 104.14) (width 1.27) (layer B.Cu) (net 1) (status 20))
 (segment (start 180.34 104.14) (end 176.53 104.14) (width 1.27) (layer B.Cu) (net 1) (status 20))
 (segment (start 156.21 104.14) (end 151.13 104.14) (width 1.27) (layer B.Cu) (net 1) (status 20))
 (segment (start 151.13 91.44) (end 154.94 91.44) (width 1.27) (layer B.Cu) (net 1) (status 10))
 (segment (start 154.94 91.44) (end 156.21 92.71) (width 1.27) (layer B.Cu) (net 1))
 (segment (start 156.21 92.71) (end 156.21 104.14) (width 1.27) (layer B.Cu) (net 1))
 (segment (start 138.43 64.77) (end 138.43 96.52) (width 1.27) (layer B.Cu) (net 1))
 (via (at 138.43 64.77) (size 2) (drill 1) (layers F.Cu B.Cu) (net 1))
 (segment (start 140.97 64.77) (end 138.43 64.77) (width 1.27) (layer F.Cu) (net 1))
 (segment (start 151.13 104.14) (end 146.05 104.14) (width 1.27) (layer B.Cu) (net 1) (status 10))
 (segment (start 146.05 104.14) (end 138.43 96.52) (width 1.27) (layer B.Cu) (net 1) (status 10))
 (segment (start 163.83 91.44) (end 167.64 91.44) (width 1.27) (layer B.Cu) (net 1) (status 10))
 (segment (start 167.64 91.44) (end 168.91 92.71) (width 1.27) (layer B.Cu) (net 1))
 (segment (start 168.91 92.71) (end 168.91 104.14) (width 1.27) (layer B.Cu) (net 1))
 (segment (start 176.53 91.44) (end 180.34 91.44) (width 1.27) (layer B.Cu) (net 1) (status 10))
 (segment (start 180.34 91.44) (end 181.61 92.71) (width 1.27) (layer B.Cu) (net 1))
 (segment (start 181.61 92.71) (end 181.61 102.87) (width 1.27) (layer B.Cu) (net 1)))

